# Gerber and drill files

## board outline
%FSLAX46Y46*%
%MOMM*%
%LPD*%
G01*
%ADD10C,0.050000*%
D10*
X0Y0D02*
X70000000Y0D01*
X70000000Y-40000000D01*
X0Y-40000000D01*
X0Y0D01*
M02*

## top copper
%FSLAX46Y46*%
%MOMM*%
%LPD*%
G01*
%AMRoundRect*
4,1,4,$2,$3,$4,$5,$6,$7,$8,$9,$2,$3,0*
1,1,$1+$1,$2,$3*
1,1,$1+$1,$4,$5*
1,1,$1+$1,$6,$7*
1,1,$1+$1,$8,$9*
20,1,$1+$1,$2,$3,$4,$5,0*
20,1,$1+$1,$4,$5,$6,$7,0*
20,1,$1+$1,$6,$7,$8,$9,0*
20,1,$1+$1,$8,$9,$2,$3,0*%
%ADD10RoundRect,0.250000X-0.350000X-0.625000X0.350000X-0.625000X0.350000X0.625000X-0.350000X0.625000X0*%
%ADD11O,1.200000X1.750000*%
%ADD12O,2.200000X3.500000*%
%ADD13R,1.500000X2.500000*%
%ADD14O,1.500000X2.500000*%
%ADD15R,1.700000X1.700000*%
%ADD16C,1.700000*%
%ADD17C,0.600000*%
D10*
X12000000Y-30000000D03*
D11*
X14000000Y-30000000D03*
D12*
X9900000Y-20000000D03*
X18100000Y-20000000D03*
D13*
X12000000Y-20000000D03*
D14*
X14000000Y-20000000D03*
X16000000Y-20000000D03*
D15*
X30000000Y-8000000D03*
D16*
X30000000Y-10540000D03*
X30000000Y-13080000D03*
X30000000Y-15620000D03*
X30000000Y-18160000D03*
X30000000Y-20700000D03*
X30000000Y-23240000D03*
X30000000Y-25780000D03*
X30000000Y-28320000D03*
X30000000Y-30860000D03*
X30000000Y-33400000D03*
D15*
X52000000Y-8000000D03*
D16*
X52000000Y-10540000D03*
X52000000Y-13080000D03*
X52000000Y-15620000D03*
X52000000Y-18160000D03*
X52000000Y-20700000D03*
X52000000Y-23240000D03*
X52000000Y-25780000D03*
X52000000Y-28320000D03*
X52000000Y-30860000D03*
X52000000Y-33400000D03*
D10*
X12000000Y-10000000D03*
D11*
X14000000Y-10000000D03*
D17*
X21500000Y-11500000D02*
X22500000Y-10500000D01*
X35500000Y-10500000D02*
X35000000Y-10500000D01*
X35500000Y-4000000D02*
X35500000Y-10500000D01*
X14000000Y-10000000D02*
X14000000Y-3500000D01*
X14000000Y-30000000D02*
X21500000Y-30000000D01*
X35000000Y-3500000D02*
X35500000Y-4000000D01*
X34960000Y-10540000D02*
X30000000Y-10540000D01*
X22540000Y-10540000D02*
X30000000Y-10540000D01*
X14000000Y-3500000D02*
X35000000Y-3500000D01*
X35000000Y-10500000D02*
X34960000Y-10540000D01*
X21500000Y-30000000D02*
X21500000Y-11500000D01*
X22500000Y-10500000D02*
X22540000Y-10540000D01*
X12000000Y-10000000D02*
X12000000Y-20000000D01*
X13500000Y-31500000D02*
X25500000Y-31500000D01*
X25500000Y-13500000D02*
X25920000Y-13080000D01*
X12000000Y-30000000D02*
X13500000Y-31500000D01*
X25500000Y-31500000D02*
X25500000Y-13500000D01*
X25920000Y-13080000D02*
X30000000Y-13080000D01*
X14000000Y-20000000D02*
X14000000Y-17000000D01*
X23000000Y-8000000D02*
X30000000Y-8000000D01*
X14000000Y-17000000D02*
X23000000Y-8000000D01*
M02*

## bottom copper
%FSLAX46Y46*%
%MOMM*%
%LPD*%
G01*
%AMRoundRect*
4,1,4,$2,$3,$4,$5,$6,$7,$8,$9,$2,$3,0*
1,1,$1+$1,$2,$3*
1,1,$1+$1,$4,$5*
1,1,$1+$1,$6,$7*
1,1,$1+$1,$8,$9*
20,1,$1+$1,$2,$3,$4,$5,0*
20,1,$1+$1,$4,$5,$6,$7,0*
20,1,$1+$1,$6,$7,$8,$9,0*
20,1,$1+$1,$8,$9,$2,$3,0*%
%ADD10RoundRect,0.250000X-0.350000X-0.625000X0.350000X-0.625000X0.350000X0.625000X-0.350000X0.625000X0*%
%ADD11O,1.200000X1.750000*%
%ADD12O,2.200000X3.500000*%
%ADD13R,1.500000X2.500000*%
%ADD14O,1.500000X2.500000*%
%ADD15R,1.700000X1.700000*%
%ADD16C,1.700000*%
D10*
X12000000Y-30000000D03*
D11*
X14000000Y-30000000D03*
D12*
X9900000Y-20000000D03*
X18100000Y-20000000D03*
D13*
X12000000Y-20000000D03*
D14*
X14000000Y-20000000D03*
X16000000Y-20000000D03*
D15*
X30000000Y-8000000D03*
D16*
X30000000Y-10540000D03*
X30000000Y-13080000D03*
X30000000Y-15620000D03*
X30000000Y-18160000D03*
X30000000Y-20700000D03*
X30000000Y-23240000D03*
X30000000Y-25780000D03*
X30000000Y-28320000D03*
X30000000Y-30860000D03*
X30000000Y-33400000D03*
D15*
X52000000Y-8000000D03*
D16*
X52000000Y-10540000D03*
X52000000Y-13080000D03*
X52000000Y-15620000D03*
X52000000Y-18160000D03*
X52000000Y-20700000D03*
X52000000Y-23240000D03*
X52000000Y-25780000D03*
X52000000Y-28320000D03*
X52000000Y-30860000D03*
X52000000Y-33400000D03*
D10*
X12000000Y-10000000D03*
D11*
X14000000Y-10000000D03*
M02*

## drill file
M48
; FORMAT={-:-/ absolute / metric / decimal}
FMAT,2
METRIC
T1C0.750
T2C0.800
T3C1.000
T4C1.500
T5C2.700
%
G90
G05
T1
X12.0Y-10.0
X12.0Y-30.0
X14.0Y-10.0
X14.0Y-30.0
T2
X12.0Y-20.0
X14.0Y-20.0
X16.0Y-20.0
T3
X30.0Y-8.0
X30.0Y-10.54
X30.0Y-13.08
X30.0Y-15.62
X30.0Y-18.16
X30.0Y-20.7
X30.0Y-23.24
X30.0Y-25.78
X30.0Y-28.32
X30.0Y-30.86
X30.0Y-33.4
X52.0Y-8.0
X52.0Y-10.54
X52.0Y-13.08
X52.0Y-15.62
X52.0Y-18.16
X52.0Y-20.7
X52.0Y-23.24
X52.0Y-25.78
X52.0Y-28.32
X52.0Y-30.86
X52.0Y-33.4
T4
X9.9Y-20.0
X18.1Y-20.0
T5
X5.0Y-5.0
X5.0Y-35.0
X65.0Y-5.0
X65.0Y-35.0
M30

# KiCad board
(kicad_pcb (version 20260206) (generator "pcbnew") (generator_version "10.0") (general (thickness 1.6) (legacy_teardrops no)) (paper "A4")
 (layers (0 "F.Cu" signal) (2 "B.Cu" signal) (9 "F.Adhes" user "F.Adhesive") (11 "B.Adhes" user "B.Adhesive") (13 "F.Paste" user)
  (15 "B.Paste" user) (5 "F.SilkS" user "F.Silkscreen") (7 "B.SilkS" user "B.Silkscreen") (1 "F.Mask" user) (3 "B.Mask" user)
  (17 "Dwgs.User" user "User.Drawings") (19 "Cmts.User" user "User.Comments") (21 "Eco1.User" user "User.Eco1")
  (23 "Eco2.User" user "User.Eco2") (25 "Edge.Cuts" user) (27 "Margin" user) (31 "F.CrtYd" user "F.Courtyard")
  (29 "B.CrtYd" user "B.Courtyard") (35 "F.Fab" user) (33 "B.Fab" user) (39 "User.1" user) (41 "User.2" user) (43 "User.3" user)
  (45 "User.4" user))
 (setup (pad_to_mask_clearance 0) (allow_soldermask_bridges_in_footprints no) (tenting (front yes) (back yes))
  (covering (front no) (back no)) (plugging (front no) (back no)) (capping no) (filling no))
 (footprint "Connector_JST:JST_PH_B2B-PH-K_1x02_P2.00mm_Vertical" (layer "F.Cu") (at 12 30)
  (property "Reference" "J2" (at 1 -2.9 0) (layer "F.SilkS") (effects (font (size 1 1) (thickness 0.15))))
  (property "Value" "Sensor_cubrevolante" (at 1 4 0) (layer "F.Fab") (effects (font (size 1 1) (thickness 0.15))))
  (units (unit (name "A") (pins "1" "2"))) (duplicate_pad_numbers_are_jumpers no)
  (pad "1" thru_hole roundrect (at 0 0) (size 1.2 1.75) (drill 0.75) (layers "*.Cu" "*.Mask") (remove_unused_layers no)
   (roundrect_rratio 0.208333) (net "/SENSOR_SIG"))
  (pad "2" thru_hole oval (at 2 0) (size 1.2 1.75) (drill 0.75) (layers "*.Cu" "*.Mask") (remove_unused_layers no) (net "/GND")))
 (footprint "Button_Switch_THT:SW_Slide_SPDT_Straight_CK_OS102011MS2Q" (layer "F.Cu") (at 12 20)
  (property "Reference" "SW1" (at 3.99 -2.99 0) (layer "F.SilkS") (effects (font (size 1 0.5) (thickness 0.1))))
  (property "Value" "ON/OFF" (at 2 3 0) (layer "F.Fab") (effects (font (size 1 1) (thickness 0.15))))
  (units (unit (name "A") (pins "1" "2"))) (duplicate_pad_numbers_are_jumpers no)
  (pad "" thru_hole oval (at -2.1 0) (size 2.2 3.5) (drill 1.5) (layers "*.Cu" "*.Mask") (remove_unused_layers no))
  (pad "" thru_hole oval (at 6.1 0) (size 2.2 3.5) (drill 1.5) (layers "*.Cu" "*.Mask") (remove_unused_layers no))
  (pad "1" thru_hole rect (at 0 0) (size 1.5 2.5) (drill 0.8) (layers "*.Cu" "*.Mask") (remove_unused_layers no) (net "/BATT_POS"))
  (pad "2" thru_hole oval (at 2 0) (size 1.5 2.5) (drill 0.8) (layers "*.Cu" "*.Mask") (remove_unused_layers no) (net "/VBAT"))
  (pad "3" thru_hole oval (at 4 0) (size 1.5 2.5) (drill 0.8) (layers "*.Cu" "*.Mask") (remove_unused_layers no)))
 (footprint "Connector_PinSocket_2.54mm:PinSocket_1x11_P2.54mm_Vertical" (layer "F.Cu") (at 30 8)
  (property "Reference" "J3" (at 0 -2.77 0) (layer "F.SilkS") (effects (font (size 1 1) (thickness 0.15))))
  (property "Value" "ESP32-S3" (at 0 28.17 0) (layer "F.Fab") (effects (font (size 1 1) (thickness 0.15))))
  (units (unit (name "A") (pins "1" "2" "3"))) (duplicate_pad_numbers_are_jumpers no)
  (pad "1" thru_hole rect (at 0 0) (size 1.7 1.7) (drill 1) (layers "*.Cu" "*.Mask") (remove_unused_layers no) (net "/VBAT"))
  (pad "2" thru_hole circle (at 0 2.54) (size 1.7 1.7) (drill 1) (layers "*.Cu" "*.Mask") (remove_unused_layers no) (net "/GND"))
  (pad "3" thru_hole circle (at 0 5.08) (size 1.7 1.7) (drill 1) (layers "*.Cu" "*.Mask") (remove_unused_layers no) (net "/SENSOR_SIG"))
  (pad "4" thru_hole circle (at 0 7.62) (size 1.7 1.7) (drill 1) (layers "*.Cu" "*.Mask") (remove_unused_layers no))
  (pad "5" thru_hole circle (at 0 10.16) (size 1.7 1.7) (drill 1) (layers "*.Cu" "*.Mask") (remove_unused_layers no))
  (pad "6" thru_hole circle (at 0 12.7) (size 1.7 1.7) (drill 1) (layers "*.Cu" "*.Mask") (remove_unused_layers no))
  (pad "7" thru_hole circle (at 0 15.24) (size 1.7 1.7) (drill 1) (layers "*.Cu" "*.Mask") (remove_unused_layers no))
  (pad "8" thru_hole circle (at 0 17.78) (size 1.7 1.7) (drill 1) (layers "*.Cu" "*.Mask") (remove_unused_layers no))
  (pad "9" thru_hole circle (at 0 20.32) (size 1.7 1.7) (drill 1) (layers "*.Cu" "*.Mask") (remove_unused_layers no))
  (pad "10" thru_hole circle (at 0 22.86) (size 1.7 1.7) (drill 1) (layers "*.Cu" "*.Mask") (remove_unused_layers no))
  (pad "11" thru_hole circle (at 0 25.4) (size 1.7 1.7) (drill 1) (layers "*.Cu" "*.Mask") (remove_unused_layers no)))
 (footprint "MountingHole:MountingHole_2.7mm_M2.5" (layer "F.Cu") (at 65 35)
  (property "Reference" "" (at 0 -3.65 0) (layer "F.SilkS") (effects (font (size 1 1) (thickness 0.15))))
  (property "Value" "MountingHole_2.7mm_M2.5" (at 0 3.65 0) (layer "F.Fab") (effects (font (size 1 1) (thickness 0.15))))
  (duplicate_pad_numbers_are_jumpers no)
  (pad "" np_thru_hole circle (at 0 0) (size 2.7 2.7) (drill 2.7) (layers "*.Cu" "*.Mask")))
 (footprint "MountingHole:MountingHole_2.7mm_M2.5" (layer "F.Cu") (at 65 5)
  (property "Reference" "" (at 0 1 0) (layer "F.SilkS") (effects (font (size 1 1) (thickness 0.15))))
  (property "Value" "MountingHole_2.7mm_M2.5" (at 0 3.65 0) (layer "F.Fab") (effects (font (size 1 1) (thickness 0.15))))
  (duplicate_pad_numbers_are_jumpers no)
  (pad "" np_thru_hole circle (at 0 0) (size 2.7 2.7) (drill 2.7) (layers "*.Cu" "*.Mask")))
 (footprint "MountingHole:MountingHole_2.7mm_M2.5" (layer "F.Cu") (at 5 5)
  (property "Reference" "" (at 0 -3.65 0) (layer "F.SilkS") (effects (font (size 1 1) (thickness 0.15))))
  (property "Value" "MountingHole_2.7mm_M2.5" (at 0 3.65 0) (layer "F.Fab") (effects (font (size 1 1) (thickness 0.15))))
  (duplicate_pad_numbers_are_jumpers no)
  (pad "" np_thru_hole circle (at 0 0) (size 2.7 2.7) (drill 2.7) (layers "*.Cu" "*.Mask")))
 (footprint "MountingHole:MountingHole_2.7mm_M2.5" (layer "F.Cu") (at 5 35)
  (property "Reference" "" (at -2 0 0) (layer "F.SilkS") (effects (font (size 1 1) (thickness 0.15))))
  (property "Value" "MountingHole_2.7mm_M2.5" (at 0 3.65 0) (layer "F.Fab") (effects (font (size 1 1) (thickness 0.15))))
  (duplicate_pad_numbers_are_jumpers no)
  (pad "" np_thru_hole circle (at 0 0) (size 2.7 2.7) (drill 2.7) (layers "*.Cu" "*.Mask")))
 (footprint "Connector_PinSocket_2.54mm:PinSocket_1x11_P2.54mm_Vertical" (layer "F.Cu") (at 52 8)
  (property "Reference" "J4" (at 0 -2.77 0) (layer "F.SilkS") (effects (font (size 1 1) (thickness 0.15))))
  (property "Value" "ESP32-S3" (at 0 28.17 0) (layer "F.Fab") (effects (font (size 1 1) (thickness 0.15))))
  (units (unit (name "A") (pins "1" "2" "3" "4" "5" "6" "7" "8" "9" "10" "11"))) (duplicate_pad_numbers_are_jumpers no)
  (pad "1" thru_hole rect (at 0 0) (size 1.7 1.7) (drill 1) (layers "*.Cu" "*.Mask") (remove_unused_layers no)
   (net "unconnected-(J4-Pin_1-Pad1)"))
  (pad "2" thru_hole circle (at 0 2.54) (size 1.7 1.7) (drill 1) (layers "*.Cu" "*.Mask") (remove_unused_layers no)
   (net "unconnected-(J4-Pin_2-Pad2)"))
  (pad "3" thru_hole circle (at 0 5.08) (size 1.7 1.7) (drill 1) (layers "*.Cu" "*.Mask") (remove_unused_layers no)
   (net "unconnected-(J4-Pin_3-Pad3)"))
  (pad "4" thru_hole circle (at 0 7.62) (size 1.7 1.7) (drill 1) (layers "*.Cu" "*.Mask") (remove_unused_layers no)
   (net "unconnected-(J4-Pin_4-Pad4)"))
  (pad "5" thru_hole circle (at 0 10.16) (size 1.7 1.7) (drill 1) (layers "*.Cu" "*.Mask") (remove_unused_layers no)
   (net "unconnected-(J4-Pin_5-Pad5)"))
  (pad "6" thru_hole circle (at 0 12.7) (size 1.7 1.7) (drill 1) (layers "*.Cu" "*.Mask") (remove_unused_layers no)
   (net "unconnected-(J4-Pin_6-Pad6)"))
  (pad "7" thru_hole circle (at 0 15.24) (size 1.7 1.7) (drill 1) (layers "*.Cu" "*.Mask") (remove_unused_layers no)
   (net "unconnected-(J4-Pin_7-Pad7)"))
  (pad "8" thru_hole circle (at 0 17.78) (size 1.7 1.7) (drill 1) (layers "*.Cu" "*.Mask") (remove_unused_layers no)
   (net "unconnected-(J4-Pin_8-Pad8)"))
  (pad "9" thru_hole circle (at 0 20.32) (size 1.7 1.7) (drill 1) (layers "*.Cu" "*.Mask") (remove_unused_layers no)
   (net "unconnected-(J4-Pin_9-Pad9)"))
  (pad "10" thru_hole circle (at 0 22.86) (size 1.7 1.7) (drill 1) (layers "*.Cu" "*.Mask") (remove_unused_layers no)
   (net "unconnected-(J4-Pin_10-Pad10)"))
  (pad "11" thru_hole circle (at 0 25.4) (size 1.7 1.7) (drill 1) (layers "*.Cu" "*.Mask") (remove_unused_layers no)
   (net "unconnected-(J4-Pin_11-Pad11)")))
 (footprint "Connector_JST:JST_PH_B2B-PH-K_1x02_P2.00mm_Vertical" (layer "F.Cu") (at 12 10)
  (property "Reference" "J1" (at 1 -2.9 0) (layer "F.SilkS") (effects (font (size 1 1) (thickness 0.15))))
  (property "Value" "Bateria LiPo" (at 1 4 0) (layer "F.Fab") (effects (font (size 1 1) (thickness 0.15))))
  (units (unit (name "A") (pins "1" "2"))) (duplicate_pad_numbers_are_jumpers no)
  (pad "1" thru_hole roundrect (at 0 0) (size 1.2 1.75) (drill 0.75) (layers "*.Cu" "*.Mask") (remove_unused_layers no)
   (roundrect_rratio 0.208333) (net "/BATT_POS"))
  (pad "2" thru_hole oval (at 2 0) (size 1.2 1.75) (drill 0.75) (layers "*.Cu" "*.Mask") (remove_unused_layers no) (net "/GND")))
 (gr_rect (start 0 0) (end 70 40) (stroke (width 0.05) (type default)) (fill no) (layer "Edge.Cuts"))
 (segment (start 21.5 11.5) (end 22.5 10.5) (width 0.6) (layer "F.Cu") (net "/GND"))
 (segment (start 35.5 10.5) (end 35 10.5) (width 0.6) (layer "F.Cu") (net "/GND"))
 (segment (start 35.5 4) (end 35.5 10.5) (width 0.6) (layer "F.Cu") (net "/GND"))
 (segment (start 14 10) (end 14 3.5) (width 0.6) (layer "F.Cu") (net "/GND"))
 (segment (start 14 30) (end 21.5 30) (width 0.6) (layer "F.Cu") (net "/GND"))
 (segment (start 35 3.5) (end 35.5 4) (width 0.6) (layer "F.Cu") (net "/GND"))
 (segment (start 34.96 10.54) (end 30 10.54) (width 0.6) (layer "F.Cu") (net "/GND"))
 (segment (start 22.54 10.54) (end 30 10.54) (width 0.6) (layer "F.Cu") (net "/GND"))
 (segment (start 14 3.5) (end 35 3.5) (width 0.6) (layer "F.Cu") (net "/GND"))
 (segment (start 35 10.5) (end 34.96 10.54) (width 0.6) (layer "F.Cu") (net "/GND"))
 (segment (start 21.5 30) (end 21.5 11.5) (width 0.6) (layer "F.Cu") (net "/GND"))
 (segment (start 22.5 10.5) (end 22.54 10.54) (width 0.6) (layer "F.Cu") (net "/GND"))
 (segment (start 12 10) (end 12 20) (width 0.6) (layer "F.Cu") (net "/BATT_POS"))
 (segment (start 13.5 31.5) (end 25.5 31.5) (width 0.6) (layer "F.Cu") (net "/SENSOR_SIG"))
 (segment (start 25.5 13.5) (end 25.92 13.08) (width 0.6) (layer "F.Cu") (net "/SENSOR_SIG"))
 (segment (start 12 30) (end 13.5 31.5) (width 0.6) (layer "F.Cu") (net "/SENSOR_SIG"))
 (segment (start 25.5 31.5) (end 25.5 13.5) (width 0.6) (layer "F.Cu") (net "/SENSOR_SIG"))
 (segment (start 25.92 13.08) (end 30 13.08) (width 0.6) (layer "F.Cu") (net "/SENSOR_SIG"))
 (segment (start 14 20) (end 14 17) (width 0.6) (layer "F.Cu") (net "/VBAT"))
 (segment (start 23 8) (end 30 8) (width 0.6) (layer "F.Cu") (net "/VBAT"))
 (segment (start 14 17) (end 23 8) (width 0.6) (layer "F.Cu") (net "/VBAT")))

